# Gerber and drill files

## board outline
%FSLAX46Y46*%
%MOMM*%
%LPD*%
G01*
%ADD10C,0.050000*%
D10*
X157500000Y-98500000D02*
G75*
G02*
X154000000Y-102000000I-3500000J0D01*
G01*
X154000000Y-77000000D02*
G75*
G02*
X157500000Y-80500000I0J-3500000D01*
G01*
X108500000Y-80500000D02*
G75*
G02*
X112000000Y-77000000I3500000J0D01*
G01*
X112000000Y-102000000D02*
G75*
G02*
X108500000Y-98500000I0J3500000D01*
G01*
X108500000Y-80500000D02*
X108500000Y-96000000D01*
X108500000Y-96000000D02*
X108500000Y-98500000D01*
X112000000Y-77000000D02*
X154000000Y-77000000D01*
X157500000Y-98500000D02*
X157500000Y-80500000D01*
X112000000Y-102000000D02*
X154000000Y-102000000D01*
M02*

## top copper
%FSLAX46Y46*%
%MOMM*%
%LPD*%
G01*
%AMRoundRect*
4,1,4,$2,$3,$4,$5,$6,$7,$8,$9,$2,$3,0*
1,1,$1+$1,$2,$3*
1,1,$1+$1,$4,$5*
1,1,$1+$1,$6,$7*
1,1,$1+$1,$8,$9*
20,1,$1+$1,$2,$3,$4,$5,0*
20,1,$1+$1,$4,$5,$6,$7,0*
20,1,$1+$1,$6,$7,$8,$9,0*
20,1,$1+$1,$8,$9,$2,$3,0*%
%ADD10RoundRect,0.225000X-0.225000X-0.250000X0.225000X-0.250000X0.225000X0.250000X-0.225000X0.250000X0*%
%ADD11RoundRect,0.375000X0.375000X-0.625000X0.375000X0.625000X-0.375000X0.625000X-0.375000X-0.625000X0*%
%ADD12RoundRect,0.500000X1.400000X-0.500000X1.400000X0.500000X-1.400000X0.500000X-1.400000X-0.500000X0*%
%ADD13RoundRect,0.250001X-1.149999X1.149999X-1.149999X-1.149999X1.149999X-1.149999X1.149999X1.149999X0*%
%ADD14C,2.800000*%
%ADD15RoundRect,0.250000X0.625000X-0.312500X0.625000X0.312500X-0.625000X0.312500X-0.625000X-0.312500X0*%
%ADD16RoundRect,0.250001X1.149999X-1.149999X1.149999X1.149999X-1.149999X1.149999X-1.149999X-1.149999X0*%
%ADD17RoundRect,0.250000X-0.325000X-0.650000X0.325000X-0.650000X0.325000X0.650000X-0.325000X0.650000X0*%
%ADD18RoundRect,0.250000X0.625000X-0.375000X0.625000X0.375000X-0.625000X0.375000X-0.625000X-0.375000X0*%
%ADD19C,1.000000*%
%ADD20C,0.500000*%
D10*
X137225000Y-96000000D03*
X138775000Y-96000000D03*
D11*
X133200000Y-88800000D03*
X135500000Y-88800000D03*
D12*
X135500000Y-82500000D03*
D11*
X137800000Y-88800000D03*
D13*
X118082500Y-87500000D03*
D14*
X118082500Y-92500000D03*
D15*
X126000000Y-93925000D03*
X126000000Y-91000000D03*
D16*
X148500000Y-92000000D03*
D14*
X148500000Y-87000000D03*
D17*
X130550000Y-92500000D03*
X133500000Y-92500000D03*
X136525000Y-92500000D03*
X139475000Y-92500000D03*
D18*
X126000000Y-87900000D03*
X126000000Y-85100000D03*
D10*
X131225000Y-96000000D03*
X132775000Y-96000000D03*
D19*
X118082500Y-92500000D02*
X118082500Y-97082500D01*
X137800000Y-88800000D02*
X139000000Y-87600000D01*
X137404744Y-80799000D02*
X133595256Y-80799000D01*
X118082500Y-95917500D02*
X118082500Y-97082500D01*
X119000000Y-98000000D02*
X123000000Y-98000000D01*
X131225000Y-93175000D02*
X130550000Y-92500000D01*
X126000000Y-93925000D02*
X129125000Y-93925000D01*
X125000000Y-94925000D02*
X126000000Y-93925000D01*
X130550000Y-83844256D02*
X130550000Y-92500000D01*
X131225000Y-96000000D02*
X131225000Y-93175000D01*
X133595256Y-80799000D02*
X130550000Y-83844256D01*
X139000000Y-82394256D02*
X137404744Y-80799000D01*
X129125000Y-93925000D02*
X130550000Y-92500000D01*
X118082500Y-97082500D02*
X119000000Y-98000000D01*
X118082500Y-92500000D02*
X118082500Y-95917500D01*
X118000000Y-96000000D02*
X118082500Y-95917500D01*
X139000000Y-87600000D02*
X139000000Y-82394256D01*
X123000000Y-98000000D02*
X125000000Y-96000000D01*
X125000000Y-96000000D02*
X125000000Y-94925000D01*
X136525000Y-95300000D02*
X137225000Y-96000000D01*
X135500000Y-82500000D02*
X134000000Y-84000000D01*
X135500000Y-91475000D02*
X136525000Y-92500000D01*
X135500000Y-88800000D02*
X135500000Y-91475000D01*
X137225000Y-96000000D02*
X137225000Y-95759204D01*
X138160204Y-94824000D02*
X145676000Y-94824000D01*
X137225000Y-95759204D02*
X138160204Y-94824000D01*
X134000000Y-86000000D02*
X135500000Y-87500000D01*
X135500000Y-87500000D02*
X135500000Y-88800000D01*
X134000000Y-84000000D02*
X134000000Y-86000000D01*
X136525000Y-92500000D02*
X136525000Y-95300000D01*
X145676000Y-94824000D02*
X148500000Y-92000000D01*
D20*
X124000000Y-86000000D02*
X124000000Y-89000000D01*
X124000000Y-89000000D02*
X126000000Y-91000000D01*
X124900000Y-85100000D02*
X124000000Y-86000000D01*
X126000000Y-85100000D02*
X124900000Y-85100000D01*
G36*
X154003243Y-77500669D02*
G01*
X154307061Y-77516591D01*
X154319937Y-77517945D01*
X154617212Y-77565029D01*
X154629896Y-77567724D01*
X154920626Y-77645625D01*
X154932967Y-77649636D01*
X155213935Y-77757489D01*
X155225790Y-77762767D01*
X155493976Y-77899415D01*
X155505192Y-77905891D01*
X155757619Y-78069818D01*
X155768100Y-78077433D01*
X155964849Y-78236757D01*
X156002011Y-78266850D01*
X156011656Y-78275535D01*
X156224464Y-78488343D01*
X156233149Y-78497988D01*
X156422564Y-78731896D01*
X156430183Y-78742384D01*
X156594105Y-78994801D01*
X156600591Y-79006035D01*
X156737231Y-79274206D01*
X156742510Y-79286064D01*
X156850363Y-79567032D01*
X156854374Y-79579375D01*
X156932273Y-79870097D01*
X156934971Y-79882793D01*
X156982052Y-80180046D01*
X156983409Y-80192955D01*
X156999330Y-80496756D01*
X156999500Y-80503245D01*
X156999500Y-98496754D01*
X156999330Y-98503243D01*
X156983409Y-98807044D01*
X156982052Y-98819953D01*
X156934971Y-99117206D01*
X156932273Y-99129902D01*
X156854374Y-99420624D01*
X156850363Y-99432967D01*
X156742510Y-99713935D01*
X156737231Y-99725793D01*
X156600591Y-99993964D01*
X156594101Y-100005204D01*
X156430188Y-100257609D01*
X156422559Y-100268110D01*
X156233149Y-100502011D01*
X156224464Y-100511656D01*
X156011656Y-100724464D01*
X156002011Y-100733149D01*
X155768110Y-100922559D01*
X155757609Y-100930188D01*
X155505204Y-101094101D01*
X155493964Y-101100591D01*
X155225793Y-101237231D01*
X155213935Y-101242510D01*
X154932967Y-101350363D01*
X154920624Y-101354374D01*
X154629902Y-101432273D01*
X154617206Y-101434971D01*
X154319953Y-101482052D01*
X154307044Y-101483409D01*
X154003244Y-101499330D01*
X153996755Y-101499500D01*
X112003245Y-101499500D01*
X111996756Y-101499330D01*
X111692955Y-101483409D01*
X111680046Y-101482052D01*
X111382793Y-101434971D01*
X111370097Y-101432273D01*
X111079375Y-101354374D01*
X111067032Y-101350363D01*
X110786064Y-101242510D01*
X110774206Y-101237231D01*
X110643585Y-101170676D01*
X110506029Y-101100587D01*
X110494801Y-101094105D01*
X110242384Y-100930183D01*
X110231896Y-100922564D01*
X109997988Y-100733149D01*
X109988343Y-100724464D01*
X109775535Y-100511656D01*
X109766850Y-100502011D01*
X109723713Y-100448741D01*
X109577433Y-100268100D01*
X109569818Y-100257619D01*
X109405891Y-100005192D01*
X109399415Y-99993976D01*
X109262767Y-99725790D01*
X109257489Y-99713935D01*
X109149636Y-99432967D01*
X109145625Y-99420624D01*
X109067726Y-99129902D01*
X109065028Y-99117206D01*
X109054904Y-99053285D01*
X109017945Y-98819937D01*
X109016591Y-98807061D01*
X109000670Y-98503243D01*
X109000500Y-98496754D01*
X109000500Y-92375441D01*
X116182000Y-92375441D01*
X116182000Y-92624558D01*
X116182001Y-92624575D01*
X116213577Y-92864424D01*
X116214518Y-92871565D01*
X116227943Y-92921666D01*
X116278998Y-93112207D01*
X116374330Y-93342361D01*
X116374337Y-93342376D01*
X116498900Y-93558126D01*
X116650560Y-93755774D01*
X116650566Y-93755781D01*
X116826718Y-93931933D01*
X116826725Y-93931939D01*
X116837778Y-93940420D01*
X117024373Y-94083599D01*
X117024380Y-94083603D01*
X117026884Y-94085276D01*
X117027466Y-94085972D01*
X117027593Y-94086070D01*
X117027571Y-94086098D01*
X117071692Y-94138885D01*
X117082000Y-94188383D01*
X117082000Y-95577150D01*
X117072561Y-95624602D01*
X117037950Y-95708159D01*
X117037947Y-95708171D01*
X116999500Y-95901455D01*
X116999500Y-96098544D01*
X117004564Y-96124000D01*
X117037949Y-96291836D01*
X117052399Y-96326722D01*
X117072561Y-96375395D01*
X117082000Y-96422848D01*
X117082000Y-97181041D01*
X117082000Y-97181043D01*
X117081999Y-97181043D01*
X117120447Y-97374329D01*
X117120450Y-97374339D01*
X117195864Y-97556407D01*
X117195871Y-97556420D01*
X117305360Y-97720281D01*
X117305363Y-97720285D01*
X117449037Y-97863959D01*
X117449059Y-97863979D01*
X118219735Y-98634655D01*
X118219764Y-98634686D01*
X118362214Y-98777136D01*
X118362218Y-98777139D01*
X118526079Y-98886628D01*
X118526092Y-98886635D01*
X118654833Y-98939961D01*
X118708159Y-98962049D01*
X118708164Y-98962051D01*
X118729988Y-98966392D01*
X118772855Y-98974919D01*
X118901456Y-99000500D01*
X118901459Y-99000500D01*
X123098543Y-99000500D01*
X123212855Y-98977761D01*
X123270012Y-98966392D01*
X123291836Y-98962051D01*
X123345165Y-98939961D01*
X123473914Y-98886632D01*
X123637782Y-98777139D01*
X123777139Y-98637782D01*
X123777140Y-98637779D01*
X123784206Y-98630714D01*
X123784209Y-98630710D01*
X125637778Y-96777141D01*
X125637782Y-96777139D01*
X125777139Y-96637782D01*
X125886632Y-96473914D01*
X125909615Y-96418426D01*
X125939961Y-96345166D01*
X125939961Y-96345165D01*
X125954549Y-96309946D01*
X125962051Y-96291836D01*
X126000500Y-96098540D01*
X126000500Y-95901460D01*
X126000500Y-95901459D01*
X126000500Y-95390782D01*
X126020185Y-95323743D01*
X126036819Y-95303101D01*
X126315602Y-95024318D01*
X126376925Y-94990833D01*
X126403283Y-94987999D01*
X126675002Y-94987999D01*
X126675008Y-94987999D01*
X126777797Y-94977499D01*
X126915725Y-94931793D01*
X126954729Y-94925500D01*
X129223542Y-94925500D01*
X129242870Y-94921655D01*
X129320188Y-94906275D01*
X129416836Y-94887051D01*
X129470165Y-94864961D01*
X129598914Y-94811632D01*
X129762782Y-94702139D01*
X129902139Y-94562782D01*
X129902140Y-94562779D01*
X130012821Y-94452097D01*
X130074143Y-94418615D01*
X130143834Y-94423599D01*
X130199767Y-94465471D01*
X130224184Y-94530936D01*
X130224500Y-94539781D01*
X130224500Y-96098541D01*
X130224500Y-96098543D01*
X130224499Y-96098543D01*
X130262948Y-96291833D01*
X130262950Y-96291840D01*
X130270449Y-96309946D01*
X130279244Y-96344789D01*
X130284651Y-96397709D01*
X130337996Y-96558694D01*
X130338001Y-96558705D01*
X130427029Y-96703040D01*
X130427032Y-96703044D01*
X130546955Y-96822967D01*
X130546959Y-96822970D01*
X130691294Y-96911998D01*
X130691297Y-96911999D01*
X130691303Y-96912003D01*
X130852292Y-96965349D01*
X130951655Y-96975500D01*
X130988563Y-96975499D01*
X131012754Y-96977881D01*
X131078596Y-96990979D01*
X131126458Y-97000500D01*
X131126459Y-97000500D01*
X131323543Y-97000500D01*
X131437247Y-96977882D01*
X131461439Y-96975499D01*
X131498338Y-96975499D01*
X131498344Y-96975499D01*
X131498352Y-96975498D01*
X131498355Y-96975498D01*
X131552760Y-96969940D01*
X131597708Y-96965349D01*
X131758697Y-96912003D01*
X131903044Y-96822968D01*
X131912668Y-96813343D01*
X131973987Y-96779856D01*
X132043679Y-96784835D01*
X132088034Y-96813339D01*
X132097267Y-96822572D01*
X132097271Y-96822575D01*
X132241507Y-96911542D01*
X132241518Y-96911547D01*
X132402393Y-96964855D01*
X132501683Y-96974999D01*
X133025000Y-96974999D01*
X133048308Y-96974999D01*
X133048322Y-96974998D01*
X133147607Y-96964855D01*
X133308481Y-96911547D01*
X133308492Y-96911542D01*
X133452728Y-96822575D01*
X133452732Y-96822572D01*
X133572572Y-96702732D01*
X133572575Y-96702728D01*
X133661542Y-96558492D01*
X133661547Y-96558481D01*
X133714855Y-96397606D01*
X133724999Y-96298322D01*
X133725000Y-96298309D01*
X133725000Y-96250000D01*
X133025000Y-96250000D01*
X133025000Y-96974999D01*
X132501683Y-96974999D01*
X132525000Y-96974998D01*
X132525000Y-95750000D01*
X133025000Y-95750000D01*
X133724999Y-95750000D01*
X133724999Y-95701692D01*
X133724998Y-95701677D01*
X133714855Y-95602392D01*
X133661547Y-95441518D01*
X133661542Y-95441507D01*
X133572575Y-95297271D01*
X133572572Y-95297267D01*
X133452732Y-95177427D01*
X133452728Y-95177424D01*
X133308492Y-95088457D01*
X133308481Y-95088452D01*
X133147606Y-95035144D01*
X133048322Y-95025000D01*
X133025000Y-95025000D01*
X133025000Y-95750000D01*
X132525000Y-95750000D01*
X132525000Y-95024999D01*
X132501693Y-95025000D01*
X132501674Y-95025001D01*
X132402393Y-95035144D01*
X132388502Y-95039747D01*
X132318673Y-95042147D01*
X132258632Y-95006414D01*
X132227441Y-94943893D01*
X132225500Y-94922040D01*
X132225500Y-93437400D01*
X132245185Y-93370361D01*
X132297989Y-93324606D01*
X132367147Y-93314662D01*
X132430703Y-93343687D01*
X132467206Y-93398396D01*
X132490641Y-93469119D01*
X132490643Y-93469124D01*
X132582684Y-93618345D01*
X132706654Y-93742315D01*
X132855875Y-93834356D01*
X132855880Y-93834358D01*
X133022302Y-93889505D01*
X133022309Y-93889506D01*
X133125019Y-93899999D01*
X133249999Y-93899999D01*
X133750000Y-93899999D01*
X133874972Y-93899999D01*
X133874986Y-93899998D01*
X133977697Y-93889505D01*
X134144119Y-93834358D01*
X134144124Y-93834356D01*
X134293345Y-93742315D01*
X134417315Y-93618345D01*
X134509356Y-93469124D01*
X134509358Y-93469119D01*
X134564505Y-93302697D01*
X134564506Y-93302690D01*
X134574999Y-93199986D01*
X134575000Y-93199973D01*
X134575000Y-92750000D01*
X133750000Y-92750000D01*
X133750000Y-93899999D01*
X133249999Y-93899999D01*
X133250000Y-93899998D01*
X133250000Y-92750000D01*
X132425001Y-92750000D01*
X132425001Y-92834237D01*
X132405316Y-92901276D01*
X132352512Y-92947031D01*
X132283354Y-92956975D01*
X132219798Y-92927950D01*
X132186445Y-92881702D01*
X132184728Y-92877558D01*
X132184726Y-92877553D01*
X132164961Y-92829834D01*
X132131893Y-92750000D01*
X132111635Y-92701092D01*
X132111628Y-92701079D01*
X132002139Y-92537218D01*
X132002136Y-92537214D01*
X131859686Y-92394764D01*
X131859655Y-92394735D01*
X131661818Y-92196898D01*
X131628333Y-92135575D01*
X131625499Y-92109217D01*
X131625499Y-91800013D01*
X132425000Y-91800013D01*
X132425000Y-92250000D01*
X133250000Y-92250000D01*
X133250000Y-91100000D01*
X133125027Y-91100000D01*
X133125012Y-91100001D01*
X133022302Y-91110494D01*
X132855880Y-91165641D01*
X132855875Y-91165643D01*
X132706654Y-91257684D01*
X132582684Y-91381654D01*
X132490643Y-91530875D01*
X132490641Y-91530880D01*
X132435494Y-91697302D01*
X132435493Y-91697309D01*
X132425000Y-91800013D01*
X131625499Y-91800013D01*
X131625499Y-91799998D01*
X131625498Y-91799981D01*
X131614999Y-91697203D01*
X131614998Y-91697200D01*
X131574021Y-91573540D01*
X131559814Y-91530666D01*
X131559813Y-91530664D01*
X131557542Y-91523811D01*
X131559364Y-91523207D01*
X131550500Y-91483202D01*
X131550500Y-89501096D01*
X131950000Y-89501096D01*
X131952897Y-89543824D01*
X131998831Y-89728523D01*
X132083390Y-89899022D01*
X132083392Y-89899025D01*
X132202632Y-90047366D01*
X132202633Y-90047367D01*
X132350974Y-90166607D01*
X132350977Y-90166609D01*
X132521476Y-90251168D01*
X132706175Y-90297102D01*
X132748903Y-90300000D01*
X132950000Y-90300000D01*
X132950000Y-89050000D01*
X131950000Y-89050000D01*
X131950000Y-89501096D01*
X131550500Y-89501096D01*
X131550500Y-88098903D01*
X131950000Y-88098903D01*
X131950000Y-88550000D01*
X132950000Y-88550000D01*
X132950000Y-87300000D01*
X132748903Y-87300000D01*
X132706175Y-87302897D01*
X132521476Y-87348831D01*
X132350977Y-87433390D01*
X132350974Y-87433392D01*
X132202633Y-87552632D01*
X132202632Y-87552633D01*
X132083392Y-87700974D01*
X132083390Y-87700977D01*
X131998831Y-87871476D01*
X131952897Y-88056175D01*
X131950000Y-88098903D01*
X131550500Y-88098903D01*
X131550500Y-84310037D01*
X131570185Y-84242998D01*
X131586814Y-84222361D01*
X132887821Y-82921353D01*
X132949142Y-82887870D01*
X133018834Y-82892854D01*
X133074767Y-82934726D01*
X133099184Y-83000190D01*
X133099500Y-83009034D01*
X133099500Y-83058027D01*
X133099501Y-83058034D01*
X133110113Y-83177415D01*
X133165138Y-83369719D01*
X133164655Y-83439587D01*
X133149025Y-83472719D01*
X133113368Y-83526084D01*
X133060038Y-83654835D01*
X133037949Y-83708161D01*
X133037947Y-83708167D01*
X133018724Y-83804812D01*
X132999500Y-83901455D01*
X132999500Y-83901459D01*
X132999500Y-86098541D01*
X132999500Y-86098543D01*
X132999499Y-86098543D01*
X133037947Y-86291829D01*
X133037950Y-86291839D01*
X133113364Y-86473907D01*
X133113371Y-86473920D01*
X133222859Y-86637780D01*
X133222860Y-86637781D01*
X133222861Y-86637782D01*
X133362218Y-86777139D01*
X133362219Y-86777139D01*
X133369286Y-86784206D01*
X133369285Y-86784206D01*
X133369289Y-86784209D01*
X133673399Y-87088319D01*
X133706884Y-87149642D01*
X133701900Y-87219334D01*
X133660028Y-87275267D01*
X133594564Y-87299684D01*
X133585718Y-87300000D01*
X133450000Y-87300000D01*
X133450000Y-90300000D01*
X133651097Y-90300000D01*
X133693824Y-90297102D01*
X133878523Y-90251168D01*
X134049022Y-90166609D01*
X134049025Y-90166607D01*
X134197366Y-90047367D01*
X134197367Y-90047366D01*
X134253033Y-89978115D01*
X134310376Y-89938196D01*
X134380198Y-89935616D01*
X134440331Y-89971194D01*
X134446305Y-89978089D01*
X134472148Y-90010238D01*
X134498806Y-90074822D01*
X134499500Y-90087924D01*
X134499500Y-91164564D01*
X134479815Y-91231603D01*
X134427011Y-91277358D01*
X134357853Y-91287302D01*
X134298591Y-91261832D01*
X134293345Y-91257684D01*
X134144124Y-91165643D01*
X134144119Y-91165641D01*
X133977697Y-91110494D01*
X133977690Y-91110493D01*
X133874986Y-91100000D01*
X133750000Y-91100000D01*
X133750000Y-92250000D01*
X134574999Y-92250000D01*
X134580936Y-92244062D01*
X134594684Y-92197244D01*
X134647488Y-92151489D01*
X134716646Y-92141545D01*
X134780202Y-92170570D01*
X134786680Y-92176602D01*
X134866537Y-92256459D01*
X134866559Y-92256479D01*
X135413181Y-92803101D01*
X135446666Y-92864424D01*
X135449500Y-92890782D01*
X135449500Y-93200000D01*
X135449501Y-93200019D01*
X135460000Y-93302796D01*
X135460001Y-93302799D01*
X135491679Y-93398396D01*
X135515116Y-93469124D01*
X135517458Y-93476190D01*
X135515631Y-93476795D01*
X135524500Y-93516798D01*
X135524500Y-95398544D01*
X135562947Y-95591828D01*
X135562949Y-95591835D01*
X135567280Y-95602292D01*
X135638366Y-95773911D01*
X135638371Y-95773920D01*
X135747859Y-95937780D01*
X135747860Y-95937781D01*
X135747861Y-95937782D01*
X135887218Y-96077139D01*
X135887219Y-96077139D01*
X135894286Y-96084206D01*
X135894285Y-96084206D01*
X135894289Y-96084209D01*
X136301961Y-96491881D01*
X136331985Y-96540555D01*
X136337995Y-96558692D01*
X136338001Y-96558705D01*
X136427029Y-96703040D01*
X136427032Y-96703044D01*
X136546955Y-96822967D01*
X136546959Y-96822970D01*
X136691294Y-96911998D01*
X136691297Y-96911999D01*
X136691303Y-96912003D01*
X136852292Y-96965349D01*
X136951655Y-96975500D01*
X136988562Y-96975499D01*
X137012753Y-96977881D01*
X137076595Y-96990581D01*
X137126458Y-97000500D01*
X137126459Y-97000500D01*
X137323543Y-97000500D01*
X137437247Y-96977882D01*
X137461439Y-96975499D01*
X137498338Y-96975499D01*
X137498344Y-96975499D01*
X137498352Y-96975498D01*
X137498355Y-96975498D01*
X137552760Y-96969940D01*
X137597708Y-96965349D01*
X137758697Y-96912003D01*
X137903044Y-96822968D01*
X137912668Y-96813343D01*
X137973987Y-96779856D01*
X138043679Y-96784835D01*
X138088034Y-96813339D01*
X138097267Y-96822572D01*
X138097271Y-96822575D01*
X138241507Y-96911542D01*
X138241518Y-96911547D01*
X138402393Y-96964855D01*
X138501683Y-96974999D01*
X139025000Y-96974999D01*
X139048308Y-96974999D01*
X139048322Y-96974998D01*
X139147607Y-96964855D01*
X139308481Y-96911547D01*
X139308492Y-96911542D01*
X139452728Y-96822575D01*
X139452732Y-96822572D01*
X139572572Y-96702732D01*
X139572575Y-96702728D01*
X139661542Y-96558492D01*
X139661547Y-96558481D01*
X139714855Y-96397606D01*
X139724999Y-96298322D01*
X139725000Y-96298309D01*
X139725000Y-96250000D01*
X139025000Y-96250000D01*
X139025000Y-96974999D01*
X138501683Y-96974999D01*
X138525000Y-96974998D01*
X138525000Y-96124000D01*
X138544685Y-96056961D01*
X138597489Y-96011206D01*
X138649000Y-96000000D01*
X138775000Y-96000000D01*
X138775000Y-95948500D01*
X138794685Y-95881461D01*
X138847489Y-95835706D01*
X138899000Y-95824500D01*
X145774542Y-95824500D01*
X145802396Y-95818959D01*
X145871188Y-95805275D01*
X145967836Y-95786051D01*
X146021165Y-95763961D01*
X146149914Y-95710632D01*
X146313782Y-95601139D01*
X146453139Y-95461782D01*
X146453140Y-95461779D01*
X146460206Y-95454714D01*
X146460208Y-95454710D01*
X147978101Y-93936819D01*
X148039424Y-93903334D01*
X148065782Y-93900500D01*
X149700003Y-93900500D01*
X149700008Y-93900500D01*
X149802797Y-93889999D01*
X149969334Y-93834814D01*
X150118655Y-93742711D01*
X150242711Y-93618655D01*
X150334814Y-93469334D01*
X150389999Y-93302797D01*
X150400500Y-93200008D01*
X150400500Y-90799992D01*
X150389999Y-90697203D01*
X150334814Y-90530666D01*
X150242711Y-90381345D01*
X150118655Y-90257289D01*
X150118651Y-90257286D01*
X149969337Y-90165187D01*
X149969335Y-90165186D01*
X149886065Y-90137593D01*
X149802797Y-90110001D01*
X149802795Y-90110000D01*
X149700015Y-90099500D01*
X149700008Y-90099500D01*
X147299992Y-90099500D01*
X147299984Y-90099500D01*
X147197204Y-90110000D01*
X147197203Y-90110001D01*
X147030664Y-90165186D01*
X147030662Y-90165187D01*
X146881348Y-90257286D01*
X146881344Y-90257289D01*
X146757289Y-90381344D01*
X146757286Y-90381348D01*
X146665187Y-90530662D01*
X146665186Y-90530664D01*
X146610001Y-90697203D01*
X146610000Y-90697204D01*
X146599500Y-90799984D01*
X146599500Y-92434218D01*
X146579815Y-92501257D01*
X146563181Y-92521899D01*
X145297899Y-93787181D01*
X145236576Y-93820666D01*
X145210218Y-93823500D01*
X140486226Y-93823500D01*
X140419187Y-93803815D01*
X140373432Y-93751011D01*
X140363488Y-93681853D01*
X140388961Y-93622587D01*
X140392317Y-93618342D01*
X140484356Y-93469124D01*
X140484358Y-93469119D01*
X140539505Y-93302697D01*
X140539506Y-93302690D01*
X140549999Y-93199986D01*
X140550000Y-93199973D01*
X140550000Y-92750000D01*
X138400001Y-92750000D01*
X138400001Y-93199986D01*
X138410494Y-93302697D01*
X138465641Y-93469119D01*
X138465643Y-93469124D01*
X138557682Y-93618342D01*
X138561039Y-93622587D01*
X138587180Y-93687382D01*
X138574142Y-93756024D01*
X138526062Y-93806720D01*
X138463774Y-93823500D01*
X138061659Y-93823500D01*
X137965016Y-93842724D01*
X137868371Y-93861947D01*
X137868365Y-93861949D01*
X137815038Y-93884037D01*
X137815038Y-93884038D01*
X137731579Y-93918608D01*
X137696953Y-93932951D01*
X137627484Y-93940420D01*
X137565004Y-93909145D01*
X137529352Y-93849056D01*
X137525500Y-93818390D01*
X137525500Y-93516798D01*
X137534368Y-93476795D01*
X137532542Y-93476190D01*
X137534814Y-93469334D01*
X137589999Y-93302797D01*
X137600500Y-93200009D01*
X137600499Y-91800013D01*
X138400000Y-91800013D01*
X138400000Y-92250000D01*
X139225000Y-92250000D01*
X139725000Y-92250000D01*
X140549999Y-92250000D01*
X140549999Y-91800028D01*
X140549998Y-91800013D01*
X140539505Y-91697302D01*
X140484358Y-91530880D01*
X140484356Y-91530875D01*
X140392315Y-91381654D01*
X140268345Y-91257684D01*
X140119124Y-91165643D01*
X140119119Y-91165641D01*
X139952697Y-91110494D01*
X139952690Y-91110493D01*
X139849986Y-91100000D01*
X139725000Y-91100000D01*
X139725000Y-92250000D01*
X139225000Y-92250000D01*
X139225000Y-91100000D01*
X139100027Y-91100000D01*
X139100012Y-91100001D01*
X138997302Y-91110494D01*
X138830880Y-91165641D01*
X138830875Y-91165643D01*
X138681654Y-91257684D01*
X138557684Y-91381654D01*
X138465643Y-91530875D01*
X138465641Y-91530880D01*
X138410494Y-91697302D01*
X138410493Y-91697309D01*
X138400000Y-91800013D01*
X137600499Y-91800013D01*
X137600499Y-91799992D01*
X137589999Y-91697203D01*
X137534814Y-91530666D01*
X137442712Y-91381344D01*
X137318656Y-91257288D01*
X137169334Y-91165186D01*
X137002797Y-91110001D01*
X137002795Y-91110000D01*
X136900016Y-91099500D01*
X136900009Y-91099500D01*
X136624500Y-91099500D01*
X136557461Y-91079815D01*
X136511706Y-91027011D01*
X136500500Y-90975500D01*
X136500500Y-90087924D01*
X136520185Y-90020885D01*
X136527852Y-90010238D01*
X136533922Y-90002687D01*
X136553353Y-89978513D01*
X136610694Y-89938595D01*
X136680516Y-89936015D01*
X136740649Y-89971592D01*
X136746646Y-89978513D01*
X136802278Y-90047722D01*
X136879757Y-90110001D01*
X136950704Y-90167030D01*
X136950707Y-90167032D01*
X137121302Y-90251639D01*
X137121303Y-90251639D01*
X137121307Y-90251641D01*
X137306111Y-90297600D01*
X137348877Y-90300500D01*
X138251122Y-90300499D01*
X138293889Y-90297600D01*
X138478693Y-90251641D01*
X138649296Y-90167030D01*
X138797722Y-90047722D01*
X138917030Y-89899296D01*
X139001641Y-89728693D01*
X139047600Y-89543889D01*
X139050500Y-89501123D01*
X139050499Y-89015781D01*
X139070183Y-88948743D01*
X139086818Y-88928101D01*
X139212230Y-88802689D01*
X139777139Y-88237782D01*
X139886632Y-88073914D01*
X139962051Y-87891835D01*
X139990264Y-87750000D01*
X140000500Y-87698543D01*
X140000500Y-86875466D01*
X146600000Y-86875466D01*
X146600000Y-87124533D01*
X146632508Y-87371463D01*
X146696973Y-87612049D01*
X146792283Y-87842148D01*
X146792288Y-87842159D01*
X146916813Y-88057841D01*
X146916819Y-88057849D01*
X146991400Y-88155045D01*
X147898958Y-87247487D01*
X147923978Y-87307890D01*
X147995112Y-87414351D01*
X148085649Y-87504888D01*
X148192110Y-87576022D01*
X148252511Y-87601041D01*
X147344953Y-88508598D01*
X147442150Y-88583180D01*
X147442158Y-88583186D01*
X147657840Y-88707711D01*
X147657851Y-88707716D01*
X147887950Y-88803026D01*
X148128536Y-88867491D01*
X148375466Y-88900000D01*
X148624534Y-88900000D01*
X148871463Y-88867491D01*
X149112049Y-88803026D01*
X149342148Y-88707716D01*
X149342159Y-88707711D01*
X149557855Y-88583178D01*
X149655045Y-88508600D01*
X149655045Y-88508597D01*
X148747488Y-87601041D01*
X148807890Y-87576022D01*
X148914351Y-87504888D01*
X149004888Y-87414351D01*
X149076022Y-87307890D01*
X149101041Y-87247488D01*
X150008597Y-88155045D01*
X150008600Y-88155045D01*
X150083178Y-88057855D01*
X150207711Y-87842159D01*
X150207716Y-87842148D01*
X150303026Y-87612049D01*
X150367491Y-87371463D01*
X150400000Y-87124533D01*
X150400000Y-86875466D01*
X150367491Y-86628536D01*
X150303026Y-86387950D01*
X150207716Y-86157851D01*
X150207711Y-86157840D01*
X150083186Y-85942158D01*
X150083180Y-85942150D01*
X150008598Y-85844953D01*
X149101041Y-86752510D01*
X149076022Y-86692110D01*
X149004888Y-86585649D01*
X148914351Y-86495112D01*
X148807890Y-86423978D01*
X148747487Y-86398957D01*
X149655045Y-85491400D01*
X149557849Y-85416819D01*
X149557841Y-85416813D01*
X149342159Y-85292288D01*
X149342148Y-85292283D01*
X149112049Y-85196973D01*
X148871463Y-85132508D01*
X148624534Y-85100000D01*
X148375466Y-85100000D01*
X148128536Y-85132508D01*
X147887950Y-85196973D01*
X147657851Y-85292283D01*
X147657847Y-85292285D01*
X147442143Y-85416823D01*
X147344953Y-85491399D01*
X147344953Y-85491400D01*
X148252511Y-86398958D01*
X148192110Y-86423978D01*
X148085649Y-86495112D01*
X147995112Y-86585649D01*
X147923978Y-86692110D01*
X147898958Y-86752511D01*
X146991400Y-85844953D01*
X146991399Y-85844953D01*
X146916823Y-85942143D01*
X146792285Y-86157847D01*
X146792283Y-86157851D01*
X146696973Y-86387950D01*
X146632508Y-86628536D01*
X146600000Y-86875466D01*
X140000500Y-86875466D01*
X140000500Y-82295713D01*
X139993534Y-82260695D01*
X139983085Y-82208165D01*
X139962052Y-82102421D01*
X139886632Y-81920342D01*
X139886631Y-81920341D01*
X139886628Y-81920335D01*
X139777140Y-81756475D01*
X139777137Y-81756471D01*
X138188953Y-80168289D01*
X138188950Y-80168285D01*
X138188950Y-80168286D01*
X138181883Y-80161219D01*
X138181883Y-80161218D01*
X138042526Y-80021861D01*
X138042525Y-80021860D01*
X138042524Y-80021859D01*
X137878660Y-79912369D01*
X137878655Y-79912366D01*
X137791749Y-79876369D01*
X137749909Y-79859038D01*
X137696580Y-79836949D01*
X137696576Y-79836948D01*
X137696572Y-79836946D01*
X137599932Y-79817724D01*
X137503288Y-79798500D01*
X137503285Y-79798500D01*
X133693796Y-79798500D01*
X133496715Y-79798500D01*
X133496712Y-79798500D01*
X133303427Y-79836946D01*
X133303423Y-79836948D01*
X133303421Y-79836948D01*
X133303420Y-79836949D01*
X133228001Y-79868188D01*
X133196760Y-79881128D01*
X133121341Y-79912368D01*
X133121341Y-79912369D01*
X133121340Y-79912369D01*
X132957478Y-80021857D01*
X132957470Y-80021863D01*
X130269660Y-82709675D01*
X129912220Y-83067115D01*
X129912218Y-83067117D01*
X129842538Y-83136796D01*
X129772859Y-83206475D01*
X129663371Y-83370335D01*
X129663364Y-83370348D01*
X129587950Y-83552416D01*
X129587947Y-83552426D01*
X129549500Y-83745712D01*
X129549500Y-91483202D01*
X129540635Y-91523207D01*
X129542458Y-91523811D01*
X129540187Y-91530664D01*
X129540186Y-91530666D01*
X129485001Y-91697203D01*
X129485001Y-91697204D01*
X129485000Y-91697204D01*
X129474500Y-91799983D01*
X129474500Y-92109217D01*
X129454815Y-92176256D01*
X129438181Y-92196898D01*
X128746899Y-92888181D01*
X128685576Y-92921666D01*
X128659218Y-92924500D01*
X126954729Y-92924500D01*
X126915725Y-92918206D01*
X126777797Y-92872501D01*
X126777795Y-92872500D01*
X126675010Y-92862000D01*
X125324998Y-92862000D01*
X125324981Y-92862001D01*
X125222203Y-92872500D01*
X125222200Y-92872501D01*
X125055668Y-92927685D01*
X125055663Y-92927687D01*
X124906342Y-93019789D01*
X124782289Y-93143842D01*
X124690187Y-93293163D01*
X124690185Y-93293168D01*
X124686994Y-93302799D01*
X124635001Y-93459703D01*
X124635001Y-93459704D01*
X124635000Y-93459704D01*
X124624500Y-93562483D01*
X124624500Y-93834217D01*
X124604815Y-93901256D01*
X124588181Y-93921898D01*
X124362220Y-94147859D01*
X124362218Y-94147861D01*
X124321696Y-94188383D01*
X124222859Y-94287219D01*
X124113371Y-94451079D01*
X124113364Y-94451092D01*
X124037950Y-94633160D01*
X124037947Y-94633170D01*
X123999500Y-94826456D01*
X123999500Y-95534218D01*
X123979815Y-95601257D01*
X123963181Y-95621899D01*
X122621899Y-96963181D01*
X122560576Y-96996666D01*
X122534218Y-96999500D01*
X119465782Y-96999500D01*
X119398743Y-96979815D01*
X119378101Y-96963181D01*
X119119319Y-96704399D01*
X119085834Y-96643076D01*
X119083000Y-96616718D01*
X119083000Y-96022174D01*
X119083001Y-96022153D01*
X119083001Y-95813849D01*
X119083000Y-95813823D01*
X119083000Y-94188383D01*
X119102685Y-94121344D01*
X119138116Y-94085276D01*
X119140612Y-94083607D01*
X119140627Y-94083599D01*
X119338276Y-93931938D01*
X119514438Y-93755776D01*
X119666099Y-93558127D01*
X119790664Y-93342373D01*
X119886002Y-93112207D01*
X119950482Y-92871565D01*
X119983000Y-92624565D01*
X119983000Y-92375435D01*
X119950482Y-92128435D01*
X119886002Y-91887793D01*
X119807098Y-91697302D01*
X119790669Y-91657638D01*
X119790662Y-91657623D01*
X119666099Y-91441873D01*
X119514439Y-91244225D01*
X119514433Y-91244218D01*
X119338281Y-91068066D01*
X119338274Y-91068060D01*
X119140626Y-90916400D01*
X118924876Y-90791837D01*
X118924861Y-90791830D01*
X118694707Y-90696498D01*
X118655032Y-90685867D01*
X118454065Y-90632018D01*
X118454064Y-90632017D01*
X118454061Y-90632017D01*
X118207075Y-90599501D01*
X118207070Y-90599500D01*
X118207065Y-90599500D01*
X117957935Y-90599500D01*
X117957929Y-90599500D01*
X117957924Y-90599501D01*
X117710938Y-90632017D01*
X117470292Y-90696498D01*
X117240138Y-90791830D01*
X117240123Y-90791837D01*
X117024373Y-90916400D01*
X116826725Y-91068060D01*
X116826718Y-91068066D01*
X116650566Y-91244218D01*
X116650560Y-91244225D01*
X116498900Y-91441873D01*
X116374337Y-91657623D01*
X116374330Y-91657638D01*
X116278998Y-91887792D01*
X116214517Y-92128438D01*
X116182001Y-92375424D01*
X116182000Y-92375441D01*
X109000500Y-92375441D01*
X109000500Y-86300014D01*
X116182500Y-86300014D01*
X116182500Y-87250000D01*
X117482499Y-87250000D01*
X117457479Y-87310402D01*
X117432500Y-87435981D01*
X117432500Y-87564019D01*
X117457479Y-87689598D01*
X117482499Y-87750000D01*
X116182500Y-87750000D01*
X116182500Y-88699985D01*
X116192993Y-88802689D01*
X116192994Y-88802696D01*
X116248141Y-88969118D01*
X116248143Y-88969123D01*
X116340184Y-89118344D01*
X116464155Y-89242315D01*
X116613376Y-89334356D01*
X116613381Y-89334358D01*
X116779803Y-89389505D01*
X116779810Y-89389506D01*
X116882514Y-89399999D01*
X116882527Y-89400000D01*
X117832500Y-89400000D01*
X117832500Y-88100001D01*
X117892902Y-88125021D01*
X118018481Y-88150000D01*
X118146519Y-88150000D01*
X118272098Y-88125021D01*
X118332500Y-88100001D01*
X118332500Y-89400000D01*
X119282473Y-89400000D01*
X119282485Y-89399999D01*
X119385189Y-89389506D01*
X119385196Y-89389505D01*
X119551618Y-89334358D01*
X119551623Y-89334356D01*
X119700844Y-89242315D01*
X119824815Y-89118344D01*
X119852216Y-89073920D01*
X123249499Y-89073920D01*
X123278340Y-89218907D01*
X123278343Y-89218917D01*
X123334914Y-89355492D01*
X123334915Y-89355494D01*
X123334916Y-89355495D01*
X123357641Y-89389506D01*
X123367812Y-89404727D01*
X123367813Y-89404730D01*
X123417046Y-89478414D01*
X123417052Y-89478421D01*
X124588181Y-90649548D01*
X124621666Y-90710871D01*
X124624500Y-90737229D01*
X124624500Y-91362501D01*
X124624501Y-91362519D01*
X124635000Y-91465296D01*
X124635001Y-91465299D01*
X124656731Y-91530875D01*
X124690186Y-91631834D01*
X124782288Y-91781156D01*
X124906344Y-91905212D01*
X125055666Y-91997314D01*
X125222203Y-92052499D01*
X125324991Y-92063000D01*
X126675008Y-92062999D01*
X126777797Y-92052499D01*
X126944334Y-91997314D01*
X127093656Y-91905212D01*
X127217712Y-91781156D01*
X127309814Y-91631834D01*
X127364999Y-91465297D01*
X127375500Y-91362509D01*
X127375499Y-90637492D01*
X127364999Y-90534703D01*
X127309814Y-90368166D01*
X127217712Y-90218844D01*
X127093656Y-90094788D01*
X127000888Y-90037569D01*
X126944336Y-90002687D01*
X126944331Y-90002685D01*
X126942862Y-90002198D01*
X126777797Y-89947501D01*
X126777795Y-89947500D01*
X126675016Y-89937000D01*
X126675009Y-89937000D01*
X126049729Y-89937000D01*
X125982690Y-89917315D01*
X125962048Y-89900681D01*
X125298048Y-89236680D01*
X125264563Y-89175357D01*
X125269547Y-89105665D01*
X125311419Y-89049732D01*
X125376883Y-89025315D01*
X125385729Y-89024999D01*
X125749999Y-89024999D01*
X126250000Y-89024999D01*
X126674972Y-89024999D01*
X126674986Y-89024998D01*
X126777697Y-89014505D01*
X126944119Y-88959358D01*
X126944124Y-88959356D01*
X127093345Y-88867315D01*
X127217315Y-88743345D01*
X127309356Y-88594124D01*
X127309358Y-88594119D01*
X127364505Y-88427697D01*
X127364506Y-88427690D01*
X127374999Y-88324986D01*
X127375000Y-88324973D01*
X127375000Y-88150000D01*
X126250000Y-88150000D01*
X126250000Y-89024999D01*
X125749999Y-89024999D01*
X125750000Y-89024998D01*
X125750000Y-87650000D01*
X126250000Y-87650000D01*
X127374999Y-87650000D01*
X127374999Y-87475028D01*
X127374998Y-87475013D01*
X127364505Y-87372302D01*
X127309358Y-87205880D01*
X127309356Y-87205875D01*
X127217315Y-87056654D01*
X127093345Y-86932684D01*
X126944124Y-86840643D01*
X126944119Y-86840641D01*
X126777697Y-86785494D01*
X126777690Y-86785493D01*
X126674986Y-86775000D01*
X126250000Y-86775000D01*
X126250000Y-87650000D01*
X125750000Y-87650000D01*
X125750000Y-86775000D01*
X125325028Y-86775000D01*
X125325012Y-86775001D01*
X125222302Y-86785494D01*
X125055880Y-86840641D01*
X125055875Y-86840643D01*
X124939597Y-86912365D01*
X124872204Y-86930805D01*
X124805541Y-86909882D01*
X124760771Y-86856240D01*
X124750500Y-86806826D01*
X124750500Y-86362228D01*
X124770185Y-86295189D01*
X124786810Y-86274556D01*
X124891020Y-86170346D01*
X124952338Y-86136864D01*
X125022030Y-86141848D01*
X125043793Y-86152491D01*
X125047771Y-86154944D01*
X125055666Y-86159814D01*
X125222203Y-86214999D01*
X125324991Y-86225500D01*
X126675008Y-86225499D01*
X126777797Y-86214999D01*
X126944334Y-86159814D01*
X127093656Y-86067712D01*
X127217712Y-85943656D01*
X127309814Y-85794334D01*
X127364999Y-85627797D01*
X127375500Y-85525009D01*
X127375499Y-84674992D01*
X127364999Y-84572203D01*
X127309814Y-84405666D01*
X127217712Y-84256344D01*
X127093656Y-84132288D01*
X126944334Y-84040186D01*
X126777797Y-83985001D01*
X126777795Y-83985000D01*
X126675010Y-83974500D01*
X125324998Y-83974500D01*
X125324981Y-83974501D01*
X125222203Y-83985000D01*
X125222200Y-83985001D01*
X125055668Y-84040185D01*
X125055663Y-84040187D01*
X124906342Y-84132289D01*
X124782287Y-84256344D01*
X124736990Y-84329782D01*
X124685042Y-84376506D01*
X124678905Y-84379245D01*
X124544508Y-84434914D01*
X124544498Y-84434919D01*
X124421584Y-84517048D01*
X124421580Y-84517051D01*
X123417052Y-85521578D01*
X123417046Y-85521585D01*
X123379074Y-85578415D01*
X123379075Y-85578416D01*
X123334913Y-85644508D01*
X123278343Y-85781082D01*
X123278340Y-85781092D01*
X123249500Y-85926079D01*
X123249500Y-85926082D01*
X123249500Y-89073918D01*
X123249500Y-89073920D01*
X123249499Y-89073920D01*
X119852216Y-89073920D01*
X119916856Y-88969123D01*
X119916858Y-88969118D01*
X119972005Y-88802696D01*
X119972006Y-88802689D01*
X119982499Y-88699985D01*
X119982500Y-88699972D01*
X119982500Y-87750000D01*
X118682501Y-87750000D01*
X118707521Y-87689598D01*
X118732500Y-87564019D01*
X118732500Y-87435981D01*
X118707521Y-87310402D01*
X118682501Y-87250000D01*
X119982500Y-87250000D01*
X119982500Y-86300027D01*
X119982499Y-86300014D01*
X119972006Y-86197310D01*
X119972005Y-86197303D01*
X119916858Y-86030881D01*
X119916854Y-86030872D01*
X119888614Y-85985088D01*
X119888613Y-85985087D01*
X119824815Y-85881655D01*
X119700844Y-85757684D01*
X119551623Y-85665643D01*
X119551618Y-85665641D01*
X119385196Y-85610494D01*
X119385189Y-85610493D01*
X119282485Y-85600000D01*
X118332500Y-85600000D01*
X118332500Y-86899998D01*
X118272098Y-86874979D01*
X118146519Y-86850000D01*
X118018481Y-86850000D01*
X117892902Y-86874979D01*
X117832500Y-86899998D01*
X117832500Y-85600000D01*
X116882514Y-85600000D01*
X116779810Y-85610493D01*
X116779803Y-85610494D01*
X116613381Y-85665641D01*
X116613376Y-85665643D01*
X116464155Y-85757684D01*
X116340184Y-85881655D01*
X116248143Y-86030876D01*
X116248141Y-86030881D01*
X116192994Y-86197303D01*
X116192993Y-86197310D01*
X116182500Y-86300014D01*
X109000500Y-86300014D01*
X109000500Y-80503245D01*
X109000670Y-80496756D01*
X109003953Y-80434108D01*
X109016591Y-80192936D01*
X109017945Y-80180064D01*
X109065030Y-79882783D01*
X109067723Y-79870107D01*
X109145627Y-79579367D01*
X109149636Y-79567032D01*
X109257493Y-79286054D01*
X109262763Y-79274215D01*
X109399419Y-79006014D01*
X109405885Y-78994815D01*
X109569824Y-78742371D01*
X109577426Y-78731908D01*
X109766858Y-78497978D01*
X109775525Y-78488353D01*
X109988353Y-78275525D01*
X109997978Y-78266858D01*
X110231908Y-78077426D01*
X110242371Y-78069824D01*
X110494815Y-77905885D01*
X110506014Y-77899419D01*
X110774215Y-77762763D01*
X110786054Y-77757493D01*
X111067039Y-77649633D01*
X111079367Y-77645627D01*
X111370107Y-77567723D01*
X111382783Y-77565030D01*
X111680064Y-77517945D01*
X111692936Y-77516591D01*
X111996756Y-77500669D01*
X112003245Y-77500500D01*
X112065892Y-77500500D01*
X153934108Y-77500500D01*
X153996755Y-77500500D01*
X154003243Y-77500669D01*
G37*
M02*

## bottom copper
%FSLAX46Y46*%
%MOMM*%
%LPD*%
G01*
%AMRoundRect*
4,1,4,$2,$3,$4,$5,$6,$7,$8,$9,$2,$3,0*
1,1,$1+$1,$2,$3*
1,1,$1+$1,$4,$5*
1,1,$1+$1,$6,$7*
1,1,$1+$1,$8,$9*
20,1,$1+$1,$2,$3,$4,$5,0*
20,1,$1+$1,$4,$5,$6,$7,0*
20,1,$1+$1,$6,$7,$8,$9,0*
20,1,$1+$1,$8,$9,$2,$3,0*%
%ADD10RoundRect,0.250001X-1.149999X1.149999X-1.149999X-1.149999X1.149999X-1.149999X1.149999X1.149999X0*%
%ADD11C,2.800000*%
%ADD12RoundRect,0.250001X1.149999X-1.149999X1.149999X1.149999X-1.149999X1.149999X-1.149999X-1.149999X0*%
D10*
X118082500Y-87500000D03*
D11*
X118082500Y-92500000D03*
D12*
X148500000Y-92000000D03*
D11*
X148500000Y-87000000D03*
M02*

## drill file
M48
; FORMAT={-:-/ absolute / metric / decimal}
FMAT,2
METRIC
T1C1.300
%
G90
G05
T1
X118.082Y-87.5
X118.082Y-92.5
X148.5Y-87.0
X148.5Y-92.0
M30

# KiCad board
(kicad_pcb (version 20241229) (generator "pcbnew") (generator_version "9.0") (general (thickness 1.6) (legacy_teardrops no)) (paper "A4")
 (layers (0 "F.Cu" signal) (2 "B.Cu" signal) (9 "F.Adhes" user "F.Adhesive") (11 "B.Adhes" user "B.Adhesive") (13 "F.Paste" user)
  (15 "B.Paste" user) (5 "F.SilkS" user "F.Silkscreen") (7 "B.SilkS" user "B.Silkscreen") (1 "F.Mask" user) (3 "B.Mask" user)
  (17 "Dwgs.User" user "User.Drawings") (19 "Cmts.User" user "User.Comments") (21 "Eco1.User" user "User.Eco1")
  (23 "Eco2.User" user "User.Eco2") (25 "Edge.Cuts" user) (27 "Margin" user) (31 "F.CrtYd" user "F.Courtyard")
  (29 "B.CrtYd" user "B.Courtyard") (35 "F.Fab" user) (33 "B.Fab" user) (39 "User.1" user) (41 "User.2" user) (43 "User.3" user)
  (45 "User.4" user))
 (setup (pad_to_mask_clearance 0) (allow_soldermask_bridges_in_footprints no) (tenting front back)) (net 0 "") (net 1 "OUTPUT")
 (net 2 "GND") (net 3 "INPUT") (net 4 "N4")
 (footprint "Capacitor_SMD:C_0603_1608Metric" (layer "F.Cu") (at 138 96)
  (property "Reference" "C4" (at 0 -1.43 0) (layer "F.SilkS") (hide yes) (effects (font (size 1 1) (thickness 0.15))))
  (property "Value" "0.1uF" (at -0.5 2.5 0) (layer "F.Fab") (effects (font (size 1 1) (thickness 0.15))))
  (pad "1" smd roundrect (at -0.775 0) (size 0.9 0.95) (layers "F.Cu" "F.Mask" "F.Paste") (roundrect_rratio 0.25) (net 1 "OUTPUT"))
  (pad "2" smd roundrect (at 0.775 0) (size 0.9 0.95) (layers "F.Cu" "F.Mask" "F.Paste") (roundrect_rratio 0.25) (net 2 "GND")))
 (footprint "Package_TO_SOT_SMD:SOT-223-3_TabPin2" (layer "F.Cu") (at 135.5 85.65 90)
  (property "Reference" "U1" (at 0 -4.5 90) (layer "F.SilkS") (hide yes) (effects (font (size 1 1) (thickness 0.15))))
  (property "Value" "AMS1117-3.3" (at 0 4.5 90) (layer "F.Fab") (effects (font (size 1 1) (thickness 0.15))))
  (pad "1" smd roundrect (at -3.15 -2.3 90) (size 2 1.5) (layers "F.Cu" "F.Mask" "F.Paste") (roundrect_rratio 0.25) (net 2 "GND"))
  (pad "2" smd roundrect (at -3.15 0 90) (size 2 1.5) (layers "F.Cu" "F.Mask" "F.Paste") (roundrect_rratio 0.25) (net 1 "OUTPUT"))
  (pad "2" smd roundrect (at 3.15 0 90) (size 2 3.8) (layers "F.Cu" "F.Mask" "F.Paste") (roundrect_rratio 0.25) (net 1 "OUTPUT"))
  (pad "3" smd roundrect (at -3.15 2.3 90) (size 2 1.5) (layers "F.Cu" "F.Mask" "F.Paste") (roundrect_rratio 0.25) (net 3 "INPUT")))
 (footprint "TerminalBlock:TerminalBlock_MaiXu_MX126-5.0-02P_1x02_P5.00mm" (layer "F.Cu") (at 118.0825 87.5 -90)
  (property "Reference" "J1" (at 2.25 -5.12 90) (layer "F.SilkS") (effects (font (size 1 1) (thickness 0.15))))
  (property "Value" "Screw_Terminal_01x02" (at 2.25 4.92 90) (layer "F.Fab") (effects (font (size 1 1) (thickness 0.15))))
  (pad "1" thru_hole roundrect (at 0 0 270) (size 2.8 2.8) (drill 1.3) (layers "*.Cu" "*.Mask") (remove_unused_layers no)
   (roundrect_rratio 0.089286) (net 2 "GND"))
  (pad "2" thru_hole circle (at 5 0 270) (size 2.8 2.8) (drill 1.3) (layers "*.Cu" "*.Mask") (remove_unused_layers no) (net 3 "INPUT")))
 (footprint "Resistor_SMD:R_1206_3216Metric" (layer "F.Cu") (at 126 92.4625 90)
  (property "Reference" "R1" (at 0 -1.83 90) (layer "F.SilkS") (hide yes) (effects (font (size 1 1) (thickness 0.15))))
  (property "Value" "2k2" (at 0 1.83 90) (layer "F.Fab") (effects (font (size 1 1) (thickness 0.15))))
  (pad "1" smd roundrect (at -1.4625 0 90) (size 1.125 1.75) (layers "F.Cu" "F.Mask" "F.Paste") (roundrect_rratio 0.222222) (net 3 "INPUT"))
  (pad "2" smd roundrect (at 1.4625 0 90) (size 1.125 1.75) (layers "F.Cu" "F.Mask" "F.Paste") (roundrect_rratio 0.222222) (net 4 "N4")))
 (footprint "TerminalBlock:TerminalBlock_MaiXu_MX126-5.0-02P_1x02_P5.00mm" (layer "F.Cu") (at 148.5 92 90)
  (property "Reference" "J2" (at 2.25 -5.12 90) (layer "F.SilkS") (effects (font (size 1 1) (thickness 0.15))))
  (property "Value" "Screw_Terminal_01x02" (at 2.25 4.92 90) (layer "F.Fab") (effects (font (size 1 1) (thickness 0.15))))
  (pad "1" thru_hole roundrect (at 0 0 90) (size 2.8 2.8) (drill 1.3) (layers "*.Cu" "*.Mask") (remove_unused_layers no)
   (roundrect_rratio 0.089286) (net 1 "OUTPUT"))
  (pad "2" thru_hole circle (at 5 0 90) (size 2.8 2.8) (drill 1.3) (layers "*.Cu" "*.Mask") (remove_unused_layers no) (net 2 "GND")))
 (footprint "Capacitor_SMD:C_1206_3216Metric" (layer "F.Cu") (at 132.025 92.5)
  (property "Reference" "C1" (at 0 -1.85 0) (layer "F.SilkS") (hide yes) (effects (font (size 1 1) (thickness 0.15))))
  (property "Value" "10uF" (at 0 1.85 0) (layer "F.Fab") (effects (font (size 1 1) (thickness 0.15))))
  (pad "1" smd roundrect (at -1.475 0) (size 1.15 1.8) (layers "F.Cu" "F.Mask" "F.Paste") (roundrect_rratio 0.217391) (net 3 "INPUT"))
  (pad "2" smd roundrect (at 1.475 0) (size 1.15 1.8) (layers "F.Cu" "F.Mask" "F.Paste") (roundrect_rratio 0.217391) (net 2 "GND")))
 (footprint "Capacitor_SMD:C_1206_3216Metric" (layer "F.Cu") (at 138 92.5)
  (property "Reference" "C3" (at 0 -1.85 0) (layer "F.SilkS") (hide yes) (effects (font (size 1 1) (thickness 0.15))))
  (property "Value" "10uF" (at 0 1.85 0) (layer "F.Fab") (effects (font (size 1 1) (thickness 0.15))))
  (pad "1" smd roundrect (at -1.475 0) (size 1.15 1.8) (layers "F.Cu" "F.Mask" "F.Paste") (roundrect_rratio 0.217391) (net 1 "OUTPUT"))
  (pad "2" smd roundrect (at 1.475 0) (size 1.15 1.8) (layers "F.Cu" "F.Mask" "F.Paste") (roundrect_rratio 0.217391) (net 2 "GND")))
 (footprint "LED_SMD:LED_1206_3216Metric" (layer "F.Cu") (at 126 86.5 90)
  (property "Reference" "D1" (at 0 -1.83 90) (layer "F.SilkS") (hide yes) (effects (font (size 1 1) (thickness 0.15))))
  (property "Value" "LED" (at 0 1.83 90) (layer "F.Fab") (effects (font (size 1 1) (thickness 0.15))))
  (pad "1" smd roundrect (at -1.4 0 90) (size 1.25 1.75) (layers "F.Cu" "F.Mask" "F.Paste") (roundrect_rratio 0.2) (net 2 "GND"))
  (pad "2" smd roundrect (at 1.4 0 90) (size 1.25 1.75) (layers "F.Cu" "F.Mask" "F.Paste") (roundrect_rratio 0.2) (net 4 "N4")))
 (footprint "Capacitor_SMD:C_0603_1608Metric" (layer "F.Cu") (at 132 96)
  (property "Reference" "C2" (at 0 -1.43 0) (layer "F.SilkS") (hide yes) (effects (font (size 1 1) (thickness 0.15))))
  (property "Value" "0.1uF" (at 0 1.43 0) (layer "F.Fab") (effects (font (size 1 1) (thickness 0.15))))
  (pad "1" smd roundrect (at -0.775 0) (size 0.9 0.95) (layers "F.Cu" "F.Mask" "F.Paste") (roundrect_rratio 0.25) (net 3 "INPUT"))
  (pad "2" smd roundrect (at 0.775 0) (size 0.9 0.95) (layers "F.Cu" "F.Mask" "F.Paste") (roundrect_rratio 0.25) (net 2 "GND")))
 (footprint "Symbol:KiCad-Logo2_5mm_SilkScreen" (layer "B.Cu") (at 130 92 180)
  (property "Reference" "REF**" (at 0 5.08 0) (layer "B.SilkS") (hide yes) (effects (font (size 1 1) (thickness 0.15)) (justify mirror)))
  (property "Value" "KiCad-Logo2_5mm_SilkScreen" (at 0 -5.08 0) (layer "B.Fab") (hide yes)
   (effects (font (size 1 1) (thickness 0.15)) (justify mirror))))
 (gr_arc (start 157.5 98.5) (mid 156.474874 100.974874) (end 154 102) (stroke (width 0.05) (type default)) (layer "Edge.Cuts"))
 (gr_arc (start 154 77) (mid 156.474874 78.025126) (end 157.5 80.5) (stroke (width 0.05) (type default)) (layer "Edge.Cuts"))
 (gr_arc (start 108.5 80.5) (mid 109.525126 78.025126) (end 112 77) (stroke (width 0.05) (type default)) (layer "Edge.Cuts"))
 (gr_arc (start 112 102) (mid 109.525126 100.974874) (end 108.5 98.5) (stroke (width 0.05) (type default)) (layer "Edge.Cuts"))
 (gr_line (start 108.5 80.5) (end 108.5 96) (stroke (width 0.05) (type default)) (layer "Edge.Cuts"))
 (gr_line (start 108.5 96) (end 108.5 98.5) (stroke (width 0.05) (type default)) (layer "Edge.Cuts"))
 (gr_line (start 112 77) (end 154 77) (stroke (width 0.05) (type default)) (layer "Edge.Cuts"))
 (gr_line (start 157.5 98.5) (end 157.5 80.5) (stroke (width 0.05) (type default)) (layer "Edge.Cuts"))
 (gr_line (start 112 102) (end 154 102) (stroke (width 0.05) (type default)) (layer "Edge.Cuts"))
 (segment (start 118.0825 92.5) (end 118.0825 97.0825) (width 1) (layer "F.Cu") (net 3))
 (segment (start 137.8 88.8) (end 139 87.6) (width 1) (layer "F.Cu") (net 3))
 (segment (start 137.404744 80.799) (end 133.595256 80.799) (width 1) (layer "F.Cu") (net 3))
 (segment (start 118.0825 95.9175) (end 118.0825 97.0825) (width 1) (layer "F.Cu") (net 3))
 (segment (start 119 98) (end 123 98) (width 1) (layer "F.Cu") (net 3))
 (segment (start 131.225 93.175) (end 130.55 92.5) (width 1) (layer "F.Cu") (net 3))
 (segment (start 126 93.925) (end 129.125 93.925) (width 1) (layer "F.Cu") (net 3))
 (segment (start 125 94.925) (end 126 93.925) (width 1) (layer "F.Cu") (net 3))
 (segment (start 130.55 83.844256) (end 130.55 92.5) (width 1) (layer "F.Cu") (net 3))
 (segment (start 131.225 96) (end 131.225 93.175) (width 1) (layer "F.Cu") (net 3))
 (segment (start 133.595256 80.799) (end 130.55 83.844256) (width 1) (layer "F.Cu") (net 3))
 (segment (start 139 82.394256) (end 137.404744 80.799) (width 1) (layer "F.Cu") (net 3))
 (segment (start 129.125 93.925) (end 130.55 92.5) (width 1) (layer "F.Cu") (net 3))
 (segment (start 118.0825 97.0825) (end 119 98) (width 1) (layer "F.Cu") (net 3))
 (segment (start 118.0825 92.5) (end 118.0825 95.9175) (width 1) (layer "F.Cu") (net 3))
 (segment (start 118 96) (end 118.0825 95.9175) (width 1) (layer "F.Cu") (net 3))
 (segment (start 139 87.6) (end 139 82.394256) (width 1) (layer "F.Cu") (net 3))
 (segment (start 123 98) (end 125 96) (width 1) (layer "F.Cu") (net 3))
 (segment (start 125 96) (end 125 94.925) (width 1) (layer "F.Cu") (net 3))
 (segment (start 136.525 95.3) (end 137.225 96) (width 1) (layer "F.Cu") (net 1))
 (segment (start 135.5 82.5) (end 134 84) (width 1) (layer "F.Cu") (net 1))
 (segment (start 135.5 91.475) (end 136.525 92.5) (width 1) (layer "F.Cu") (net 1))
 (segment (start 135.5 88.8) (end 135.5 91.475) (width 1) (layer "F.Cu") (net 1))
 (segment (start 137.225 96) (end 137.225 95.759204) (width 1) (layer "F.Cu") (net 1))
 (segment (start 138.160204 94.824) (end 145.676 94.824) (width 1) (layer "F.Cu") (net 1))
 (segment (start 137.225 95.759204) (end 138.160204 94.824) (width 1) (layer "F.Cu") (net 1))
 (segment (start 134 86) (end 135.5 87.5) (width 1) (layer "F.Cu") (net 1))
 (segment (start 135.5 87.5) (end 135.5 88.8) (width 1) (layer "F.Cu") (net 1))
 (segment (start 134 84) (end 134 86) (width 1) (layer "F.Cu") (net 1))
 (segment (start 136.525 92.5) (end 136.525 95.3) (width 1) (layer "F.Cu") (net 1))
 (segment (start 145.676 94.824) (end 148.5 92) (width 1) (layer "F.Cu") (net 1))
 (segment (start 124 86) (end 124 89) (width 0.5) (layer "F.Cu") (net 4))
 (segment (start 124 89) (end 126 91) (width 0.5) (layer "F.Cu") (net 4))
 (segment (start 124.9 85.1) (end 124 86) (width 0.5) (layer "F.Cu") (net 4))
 (segment (start 126 85.1) (end 124.9 85.1) (width 0.5) (layer "F.Cu") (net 4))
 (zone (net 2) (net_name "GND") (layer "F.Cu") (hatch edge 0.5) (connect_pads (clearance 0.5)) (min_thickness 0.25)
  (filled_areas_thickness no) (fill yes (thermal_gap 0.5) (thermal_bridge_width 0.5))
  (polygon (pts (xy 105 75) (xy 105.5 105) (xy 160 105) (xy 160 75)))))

